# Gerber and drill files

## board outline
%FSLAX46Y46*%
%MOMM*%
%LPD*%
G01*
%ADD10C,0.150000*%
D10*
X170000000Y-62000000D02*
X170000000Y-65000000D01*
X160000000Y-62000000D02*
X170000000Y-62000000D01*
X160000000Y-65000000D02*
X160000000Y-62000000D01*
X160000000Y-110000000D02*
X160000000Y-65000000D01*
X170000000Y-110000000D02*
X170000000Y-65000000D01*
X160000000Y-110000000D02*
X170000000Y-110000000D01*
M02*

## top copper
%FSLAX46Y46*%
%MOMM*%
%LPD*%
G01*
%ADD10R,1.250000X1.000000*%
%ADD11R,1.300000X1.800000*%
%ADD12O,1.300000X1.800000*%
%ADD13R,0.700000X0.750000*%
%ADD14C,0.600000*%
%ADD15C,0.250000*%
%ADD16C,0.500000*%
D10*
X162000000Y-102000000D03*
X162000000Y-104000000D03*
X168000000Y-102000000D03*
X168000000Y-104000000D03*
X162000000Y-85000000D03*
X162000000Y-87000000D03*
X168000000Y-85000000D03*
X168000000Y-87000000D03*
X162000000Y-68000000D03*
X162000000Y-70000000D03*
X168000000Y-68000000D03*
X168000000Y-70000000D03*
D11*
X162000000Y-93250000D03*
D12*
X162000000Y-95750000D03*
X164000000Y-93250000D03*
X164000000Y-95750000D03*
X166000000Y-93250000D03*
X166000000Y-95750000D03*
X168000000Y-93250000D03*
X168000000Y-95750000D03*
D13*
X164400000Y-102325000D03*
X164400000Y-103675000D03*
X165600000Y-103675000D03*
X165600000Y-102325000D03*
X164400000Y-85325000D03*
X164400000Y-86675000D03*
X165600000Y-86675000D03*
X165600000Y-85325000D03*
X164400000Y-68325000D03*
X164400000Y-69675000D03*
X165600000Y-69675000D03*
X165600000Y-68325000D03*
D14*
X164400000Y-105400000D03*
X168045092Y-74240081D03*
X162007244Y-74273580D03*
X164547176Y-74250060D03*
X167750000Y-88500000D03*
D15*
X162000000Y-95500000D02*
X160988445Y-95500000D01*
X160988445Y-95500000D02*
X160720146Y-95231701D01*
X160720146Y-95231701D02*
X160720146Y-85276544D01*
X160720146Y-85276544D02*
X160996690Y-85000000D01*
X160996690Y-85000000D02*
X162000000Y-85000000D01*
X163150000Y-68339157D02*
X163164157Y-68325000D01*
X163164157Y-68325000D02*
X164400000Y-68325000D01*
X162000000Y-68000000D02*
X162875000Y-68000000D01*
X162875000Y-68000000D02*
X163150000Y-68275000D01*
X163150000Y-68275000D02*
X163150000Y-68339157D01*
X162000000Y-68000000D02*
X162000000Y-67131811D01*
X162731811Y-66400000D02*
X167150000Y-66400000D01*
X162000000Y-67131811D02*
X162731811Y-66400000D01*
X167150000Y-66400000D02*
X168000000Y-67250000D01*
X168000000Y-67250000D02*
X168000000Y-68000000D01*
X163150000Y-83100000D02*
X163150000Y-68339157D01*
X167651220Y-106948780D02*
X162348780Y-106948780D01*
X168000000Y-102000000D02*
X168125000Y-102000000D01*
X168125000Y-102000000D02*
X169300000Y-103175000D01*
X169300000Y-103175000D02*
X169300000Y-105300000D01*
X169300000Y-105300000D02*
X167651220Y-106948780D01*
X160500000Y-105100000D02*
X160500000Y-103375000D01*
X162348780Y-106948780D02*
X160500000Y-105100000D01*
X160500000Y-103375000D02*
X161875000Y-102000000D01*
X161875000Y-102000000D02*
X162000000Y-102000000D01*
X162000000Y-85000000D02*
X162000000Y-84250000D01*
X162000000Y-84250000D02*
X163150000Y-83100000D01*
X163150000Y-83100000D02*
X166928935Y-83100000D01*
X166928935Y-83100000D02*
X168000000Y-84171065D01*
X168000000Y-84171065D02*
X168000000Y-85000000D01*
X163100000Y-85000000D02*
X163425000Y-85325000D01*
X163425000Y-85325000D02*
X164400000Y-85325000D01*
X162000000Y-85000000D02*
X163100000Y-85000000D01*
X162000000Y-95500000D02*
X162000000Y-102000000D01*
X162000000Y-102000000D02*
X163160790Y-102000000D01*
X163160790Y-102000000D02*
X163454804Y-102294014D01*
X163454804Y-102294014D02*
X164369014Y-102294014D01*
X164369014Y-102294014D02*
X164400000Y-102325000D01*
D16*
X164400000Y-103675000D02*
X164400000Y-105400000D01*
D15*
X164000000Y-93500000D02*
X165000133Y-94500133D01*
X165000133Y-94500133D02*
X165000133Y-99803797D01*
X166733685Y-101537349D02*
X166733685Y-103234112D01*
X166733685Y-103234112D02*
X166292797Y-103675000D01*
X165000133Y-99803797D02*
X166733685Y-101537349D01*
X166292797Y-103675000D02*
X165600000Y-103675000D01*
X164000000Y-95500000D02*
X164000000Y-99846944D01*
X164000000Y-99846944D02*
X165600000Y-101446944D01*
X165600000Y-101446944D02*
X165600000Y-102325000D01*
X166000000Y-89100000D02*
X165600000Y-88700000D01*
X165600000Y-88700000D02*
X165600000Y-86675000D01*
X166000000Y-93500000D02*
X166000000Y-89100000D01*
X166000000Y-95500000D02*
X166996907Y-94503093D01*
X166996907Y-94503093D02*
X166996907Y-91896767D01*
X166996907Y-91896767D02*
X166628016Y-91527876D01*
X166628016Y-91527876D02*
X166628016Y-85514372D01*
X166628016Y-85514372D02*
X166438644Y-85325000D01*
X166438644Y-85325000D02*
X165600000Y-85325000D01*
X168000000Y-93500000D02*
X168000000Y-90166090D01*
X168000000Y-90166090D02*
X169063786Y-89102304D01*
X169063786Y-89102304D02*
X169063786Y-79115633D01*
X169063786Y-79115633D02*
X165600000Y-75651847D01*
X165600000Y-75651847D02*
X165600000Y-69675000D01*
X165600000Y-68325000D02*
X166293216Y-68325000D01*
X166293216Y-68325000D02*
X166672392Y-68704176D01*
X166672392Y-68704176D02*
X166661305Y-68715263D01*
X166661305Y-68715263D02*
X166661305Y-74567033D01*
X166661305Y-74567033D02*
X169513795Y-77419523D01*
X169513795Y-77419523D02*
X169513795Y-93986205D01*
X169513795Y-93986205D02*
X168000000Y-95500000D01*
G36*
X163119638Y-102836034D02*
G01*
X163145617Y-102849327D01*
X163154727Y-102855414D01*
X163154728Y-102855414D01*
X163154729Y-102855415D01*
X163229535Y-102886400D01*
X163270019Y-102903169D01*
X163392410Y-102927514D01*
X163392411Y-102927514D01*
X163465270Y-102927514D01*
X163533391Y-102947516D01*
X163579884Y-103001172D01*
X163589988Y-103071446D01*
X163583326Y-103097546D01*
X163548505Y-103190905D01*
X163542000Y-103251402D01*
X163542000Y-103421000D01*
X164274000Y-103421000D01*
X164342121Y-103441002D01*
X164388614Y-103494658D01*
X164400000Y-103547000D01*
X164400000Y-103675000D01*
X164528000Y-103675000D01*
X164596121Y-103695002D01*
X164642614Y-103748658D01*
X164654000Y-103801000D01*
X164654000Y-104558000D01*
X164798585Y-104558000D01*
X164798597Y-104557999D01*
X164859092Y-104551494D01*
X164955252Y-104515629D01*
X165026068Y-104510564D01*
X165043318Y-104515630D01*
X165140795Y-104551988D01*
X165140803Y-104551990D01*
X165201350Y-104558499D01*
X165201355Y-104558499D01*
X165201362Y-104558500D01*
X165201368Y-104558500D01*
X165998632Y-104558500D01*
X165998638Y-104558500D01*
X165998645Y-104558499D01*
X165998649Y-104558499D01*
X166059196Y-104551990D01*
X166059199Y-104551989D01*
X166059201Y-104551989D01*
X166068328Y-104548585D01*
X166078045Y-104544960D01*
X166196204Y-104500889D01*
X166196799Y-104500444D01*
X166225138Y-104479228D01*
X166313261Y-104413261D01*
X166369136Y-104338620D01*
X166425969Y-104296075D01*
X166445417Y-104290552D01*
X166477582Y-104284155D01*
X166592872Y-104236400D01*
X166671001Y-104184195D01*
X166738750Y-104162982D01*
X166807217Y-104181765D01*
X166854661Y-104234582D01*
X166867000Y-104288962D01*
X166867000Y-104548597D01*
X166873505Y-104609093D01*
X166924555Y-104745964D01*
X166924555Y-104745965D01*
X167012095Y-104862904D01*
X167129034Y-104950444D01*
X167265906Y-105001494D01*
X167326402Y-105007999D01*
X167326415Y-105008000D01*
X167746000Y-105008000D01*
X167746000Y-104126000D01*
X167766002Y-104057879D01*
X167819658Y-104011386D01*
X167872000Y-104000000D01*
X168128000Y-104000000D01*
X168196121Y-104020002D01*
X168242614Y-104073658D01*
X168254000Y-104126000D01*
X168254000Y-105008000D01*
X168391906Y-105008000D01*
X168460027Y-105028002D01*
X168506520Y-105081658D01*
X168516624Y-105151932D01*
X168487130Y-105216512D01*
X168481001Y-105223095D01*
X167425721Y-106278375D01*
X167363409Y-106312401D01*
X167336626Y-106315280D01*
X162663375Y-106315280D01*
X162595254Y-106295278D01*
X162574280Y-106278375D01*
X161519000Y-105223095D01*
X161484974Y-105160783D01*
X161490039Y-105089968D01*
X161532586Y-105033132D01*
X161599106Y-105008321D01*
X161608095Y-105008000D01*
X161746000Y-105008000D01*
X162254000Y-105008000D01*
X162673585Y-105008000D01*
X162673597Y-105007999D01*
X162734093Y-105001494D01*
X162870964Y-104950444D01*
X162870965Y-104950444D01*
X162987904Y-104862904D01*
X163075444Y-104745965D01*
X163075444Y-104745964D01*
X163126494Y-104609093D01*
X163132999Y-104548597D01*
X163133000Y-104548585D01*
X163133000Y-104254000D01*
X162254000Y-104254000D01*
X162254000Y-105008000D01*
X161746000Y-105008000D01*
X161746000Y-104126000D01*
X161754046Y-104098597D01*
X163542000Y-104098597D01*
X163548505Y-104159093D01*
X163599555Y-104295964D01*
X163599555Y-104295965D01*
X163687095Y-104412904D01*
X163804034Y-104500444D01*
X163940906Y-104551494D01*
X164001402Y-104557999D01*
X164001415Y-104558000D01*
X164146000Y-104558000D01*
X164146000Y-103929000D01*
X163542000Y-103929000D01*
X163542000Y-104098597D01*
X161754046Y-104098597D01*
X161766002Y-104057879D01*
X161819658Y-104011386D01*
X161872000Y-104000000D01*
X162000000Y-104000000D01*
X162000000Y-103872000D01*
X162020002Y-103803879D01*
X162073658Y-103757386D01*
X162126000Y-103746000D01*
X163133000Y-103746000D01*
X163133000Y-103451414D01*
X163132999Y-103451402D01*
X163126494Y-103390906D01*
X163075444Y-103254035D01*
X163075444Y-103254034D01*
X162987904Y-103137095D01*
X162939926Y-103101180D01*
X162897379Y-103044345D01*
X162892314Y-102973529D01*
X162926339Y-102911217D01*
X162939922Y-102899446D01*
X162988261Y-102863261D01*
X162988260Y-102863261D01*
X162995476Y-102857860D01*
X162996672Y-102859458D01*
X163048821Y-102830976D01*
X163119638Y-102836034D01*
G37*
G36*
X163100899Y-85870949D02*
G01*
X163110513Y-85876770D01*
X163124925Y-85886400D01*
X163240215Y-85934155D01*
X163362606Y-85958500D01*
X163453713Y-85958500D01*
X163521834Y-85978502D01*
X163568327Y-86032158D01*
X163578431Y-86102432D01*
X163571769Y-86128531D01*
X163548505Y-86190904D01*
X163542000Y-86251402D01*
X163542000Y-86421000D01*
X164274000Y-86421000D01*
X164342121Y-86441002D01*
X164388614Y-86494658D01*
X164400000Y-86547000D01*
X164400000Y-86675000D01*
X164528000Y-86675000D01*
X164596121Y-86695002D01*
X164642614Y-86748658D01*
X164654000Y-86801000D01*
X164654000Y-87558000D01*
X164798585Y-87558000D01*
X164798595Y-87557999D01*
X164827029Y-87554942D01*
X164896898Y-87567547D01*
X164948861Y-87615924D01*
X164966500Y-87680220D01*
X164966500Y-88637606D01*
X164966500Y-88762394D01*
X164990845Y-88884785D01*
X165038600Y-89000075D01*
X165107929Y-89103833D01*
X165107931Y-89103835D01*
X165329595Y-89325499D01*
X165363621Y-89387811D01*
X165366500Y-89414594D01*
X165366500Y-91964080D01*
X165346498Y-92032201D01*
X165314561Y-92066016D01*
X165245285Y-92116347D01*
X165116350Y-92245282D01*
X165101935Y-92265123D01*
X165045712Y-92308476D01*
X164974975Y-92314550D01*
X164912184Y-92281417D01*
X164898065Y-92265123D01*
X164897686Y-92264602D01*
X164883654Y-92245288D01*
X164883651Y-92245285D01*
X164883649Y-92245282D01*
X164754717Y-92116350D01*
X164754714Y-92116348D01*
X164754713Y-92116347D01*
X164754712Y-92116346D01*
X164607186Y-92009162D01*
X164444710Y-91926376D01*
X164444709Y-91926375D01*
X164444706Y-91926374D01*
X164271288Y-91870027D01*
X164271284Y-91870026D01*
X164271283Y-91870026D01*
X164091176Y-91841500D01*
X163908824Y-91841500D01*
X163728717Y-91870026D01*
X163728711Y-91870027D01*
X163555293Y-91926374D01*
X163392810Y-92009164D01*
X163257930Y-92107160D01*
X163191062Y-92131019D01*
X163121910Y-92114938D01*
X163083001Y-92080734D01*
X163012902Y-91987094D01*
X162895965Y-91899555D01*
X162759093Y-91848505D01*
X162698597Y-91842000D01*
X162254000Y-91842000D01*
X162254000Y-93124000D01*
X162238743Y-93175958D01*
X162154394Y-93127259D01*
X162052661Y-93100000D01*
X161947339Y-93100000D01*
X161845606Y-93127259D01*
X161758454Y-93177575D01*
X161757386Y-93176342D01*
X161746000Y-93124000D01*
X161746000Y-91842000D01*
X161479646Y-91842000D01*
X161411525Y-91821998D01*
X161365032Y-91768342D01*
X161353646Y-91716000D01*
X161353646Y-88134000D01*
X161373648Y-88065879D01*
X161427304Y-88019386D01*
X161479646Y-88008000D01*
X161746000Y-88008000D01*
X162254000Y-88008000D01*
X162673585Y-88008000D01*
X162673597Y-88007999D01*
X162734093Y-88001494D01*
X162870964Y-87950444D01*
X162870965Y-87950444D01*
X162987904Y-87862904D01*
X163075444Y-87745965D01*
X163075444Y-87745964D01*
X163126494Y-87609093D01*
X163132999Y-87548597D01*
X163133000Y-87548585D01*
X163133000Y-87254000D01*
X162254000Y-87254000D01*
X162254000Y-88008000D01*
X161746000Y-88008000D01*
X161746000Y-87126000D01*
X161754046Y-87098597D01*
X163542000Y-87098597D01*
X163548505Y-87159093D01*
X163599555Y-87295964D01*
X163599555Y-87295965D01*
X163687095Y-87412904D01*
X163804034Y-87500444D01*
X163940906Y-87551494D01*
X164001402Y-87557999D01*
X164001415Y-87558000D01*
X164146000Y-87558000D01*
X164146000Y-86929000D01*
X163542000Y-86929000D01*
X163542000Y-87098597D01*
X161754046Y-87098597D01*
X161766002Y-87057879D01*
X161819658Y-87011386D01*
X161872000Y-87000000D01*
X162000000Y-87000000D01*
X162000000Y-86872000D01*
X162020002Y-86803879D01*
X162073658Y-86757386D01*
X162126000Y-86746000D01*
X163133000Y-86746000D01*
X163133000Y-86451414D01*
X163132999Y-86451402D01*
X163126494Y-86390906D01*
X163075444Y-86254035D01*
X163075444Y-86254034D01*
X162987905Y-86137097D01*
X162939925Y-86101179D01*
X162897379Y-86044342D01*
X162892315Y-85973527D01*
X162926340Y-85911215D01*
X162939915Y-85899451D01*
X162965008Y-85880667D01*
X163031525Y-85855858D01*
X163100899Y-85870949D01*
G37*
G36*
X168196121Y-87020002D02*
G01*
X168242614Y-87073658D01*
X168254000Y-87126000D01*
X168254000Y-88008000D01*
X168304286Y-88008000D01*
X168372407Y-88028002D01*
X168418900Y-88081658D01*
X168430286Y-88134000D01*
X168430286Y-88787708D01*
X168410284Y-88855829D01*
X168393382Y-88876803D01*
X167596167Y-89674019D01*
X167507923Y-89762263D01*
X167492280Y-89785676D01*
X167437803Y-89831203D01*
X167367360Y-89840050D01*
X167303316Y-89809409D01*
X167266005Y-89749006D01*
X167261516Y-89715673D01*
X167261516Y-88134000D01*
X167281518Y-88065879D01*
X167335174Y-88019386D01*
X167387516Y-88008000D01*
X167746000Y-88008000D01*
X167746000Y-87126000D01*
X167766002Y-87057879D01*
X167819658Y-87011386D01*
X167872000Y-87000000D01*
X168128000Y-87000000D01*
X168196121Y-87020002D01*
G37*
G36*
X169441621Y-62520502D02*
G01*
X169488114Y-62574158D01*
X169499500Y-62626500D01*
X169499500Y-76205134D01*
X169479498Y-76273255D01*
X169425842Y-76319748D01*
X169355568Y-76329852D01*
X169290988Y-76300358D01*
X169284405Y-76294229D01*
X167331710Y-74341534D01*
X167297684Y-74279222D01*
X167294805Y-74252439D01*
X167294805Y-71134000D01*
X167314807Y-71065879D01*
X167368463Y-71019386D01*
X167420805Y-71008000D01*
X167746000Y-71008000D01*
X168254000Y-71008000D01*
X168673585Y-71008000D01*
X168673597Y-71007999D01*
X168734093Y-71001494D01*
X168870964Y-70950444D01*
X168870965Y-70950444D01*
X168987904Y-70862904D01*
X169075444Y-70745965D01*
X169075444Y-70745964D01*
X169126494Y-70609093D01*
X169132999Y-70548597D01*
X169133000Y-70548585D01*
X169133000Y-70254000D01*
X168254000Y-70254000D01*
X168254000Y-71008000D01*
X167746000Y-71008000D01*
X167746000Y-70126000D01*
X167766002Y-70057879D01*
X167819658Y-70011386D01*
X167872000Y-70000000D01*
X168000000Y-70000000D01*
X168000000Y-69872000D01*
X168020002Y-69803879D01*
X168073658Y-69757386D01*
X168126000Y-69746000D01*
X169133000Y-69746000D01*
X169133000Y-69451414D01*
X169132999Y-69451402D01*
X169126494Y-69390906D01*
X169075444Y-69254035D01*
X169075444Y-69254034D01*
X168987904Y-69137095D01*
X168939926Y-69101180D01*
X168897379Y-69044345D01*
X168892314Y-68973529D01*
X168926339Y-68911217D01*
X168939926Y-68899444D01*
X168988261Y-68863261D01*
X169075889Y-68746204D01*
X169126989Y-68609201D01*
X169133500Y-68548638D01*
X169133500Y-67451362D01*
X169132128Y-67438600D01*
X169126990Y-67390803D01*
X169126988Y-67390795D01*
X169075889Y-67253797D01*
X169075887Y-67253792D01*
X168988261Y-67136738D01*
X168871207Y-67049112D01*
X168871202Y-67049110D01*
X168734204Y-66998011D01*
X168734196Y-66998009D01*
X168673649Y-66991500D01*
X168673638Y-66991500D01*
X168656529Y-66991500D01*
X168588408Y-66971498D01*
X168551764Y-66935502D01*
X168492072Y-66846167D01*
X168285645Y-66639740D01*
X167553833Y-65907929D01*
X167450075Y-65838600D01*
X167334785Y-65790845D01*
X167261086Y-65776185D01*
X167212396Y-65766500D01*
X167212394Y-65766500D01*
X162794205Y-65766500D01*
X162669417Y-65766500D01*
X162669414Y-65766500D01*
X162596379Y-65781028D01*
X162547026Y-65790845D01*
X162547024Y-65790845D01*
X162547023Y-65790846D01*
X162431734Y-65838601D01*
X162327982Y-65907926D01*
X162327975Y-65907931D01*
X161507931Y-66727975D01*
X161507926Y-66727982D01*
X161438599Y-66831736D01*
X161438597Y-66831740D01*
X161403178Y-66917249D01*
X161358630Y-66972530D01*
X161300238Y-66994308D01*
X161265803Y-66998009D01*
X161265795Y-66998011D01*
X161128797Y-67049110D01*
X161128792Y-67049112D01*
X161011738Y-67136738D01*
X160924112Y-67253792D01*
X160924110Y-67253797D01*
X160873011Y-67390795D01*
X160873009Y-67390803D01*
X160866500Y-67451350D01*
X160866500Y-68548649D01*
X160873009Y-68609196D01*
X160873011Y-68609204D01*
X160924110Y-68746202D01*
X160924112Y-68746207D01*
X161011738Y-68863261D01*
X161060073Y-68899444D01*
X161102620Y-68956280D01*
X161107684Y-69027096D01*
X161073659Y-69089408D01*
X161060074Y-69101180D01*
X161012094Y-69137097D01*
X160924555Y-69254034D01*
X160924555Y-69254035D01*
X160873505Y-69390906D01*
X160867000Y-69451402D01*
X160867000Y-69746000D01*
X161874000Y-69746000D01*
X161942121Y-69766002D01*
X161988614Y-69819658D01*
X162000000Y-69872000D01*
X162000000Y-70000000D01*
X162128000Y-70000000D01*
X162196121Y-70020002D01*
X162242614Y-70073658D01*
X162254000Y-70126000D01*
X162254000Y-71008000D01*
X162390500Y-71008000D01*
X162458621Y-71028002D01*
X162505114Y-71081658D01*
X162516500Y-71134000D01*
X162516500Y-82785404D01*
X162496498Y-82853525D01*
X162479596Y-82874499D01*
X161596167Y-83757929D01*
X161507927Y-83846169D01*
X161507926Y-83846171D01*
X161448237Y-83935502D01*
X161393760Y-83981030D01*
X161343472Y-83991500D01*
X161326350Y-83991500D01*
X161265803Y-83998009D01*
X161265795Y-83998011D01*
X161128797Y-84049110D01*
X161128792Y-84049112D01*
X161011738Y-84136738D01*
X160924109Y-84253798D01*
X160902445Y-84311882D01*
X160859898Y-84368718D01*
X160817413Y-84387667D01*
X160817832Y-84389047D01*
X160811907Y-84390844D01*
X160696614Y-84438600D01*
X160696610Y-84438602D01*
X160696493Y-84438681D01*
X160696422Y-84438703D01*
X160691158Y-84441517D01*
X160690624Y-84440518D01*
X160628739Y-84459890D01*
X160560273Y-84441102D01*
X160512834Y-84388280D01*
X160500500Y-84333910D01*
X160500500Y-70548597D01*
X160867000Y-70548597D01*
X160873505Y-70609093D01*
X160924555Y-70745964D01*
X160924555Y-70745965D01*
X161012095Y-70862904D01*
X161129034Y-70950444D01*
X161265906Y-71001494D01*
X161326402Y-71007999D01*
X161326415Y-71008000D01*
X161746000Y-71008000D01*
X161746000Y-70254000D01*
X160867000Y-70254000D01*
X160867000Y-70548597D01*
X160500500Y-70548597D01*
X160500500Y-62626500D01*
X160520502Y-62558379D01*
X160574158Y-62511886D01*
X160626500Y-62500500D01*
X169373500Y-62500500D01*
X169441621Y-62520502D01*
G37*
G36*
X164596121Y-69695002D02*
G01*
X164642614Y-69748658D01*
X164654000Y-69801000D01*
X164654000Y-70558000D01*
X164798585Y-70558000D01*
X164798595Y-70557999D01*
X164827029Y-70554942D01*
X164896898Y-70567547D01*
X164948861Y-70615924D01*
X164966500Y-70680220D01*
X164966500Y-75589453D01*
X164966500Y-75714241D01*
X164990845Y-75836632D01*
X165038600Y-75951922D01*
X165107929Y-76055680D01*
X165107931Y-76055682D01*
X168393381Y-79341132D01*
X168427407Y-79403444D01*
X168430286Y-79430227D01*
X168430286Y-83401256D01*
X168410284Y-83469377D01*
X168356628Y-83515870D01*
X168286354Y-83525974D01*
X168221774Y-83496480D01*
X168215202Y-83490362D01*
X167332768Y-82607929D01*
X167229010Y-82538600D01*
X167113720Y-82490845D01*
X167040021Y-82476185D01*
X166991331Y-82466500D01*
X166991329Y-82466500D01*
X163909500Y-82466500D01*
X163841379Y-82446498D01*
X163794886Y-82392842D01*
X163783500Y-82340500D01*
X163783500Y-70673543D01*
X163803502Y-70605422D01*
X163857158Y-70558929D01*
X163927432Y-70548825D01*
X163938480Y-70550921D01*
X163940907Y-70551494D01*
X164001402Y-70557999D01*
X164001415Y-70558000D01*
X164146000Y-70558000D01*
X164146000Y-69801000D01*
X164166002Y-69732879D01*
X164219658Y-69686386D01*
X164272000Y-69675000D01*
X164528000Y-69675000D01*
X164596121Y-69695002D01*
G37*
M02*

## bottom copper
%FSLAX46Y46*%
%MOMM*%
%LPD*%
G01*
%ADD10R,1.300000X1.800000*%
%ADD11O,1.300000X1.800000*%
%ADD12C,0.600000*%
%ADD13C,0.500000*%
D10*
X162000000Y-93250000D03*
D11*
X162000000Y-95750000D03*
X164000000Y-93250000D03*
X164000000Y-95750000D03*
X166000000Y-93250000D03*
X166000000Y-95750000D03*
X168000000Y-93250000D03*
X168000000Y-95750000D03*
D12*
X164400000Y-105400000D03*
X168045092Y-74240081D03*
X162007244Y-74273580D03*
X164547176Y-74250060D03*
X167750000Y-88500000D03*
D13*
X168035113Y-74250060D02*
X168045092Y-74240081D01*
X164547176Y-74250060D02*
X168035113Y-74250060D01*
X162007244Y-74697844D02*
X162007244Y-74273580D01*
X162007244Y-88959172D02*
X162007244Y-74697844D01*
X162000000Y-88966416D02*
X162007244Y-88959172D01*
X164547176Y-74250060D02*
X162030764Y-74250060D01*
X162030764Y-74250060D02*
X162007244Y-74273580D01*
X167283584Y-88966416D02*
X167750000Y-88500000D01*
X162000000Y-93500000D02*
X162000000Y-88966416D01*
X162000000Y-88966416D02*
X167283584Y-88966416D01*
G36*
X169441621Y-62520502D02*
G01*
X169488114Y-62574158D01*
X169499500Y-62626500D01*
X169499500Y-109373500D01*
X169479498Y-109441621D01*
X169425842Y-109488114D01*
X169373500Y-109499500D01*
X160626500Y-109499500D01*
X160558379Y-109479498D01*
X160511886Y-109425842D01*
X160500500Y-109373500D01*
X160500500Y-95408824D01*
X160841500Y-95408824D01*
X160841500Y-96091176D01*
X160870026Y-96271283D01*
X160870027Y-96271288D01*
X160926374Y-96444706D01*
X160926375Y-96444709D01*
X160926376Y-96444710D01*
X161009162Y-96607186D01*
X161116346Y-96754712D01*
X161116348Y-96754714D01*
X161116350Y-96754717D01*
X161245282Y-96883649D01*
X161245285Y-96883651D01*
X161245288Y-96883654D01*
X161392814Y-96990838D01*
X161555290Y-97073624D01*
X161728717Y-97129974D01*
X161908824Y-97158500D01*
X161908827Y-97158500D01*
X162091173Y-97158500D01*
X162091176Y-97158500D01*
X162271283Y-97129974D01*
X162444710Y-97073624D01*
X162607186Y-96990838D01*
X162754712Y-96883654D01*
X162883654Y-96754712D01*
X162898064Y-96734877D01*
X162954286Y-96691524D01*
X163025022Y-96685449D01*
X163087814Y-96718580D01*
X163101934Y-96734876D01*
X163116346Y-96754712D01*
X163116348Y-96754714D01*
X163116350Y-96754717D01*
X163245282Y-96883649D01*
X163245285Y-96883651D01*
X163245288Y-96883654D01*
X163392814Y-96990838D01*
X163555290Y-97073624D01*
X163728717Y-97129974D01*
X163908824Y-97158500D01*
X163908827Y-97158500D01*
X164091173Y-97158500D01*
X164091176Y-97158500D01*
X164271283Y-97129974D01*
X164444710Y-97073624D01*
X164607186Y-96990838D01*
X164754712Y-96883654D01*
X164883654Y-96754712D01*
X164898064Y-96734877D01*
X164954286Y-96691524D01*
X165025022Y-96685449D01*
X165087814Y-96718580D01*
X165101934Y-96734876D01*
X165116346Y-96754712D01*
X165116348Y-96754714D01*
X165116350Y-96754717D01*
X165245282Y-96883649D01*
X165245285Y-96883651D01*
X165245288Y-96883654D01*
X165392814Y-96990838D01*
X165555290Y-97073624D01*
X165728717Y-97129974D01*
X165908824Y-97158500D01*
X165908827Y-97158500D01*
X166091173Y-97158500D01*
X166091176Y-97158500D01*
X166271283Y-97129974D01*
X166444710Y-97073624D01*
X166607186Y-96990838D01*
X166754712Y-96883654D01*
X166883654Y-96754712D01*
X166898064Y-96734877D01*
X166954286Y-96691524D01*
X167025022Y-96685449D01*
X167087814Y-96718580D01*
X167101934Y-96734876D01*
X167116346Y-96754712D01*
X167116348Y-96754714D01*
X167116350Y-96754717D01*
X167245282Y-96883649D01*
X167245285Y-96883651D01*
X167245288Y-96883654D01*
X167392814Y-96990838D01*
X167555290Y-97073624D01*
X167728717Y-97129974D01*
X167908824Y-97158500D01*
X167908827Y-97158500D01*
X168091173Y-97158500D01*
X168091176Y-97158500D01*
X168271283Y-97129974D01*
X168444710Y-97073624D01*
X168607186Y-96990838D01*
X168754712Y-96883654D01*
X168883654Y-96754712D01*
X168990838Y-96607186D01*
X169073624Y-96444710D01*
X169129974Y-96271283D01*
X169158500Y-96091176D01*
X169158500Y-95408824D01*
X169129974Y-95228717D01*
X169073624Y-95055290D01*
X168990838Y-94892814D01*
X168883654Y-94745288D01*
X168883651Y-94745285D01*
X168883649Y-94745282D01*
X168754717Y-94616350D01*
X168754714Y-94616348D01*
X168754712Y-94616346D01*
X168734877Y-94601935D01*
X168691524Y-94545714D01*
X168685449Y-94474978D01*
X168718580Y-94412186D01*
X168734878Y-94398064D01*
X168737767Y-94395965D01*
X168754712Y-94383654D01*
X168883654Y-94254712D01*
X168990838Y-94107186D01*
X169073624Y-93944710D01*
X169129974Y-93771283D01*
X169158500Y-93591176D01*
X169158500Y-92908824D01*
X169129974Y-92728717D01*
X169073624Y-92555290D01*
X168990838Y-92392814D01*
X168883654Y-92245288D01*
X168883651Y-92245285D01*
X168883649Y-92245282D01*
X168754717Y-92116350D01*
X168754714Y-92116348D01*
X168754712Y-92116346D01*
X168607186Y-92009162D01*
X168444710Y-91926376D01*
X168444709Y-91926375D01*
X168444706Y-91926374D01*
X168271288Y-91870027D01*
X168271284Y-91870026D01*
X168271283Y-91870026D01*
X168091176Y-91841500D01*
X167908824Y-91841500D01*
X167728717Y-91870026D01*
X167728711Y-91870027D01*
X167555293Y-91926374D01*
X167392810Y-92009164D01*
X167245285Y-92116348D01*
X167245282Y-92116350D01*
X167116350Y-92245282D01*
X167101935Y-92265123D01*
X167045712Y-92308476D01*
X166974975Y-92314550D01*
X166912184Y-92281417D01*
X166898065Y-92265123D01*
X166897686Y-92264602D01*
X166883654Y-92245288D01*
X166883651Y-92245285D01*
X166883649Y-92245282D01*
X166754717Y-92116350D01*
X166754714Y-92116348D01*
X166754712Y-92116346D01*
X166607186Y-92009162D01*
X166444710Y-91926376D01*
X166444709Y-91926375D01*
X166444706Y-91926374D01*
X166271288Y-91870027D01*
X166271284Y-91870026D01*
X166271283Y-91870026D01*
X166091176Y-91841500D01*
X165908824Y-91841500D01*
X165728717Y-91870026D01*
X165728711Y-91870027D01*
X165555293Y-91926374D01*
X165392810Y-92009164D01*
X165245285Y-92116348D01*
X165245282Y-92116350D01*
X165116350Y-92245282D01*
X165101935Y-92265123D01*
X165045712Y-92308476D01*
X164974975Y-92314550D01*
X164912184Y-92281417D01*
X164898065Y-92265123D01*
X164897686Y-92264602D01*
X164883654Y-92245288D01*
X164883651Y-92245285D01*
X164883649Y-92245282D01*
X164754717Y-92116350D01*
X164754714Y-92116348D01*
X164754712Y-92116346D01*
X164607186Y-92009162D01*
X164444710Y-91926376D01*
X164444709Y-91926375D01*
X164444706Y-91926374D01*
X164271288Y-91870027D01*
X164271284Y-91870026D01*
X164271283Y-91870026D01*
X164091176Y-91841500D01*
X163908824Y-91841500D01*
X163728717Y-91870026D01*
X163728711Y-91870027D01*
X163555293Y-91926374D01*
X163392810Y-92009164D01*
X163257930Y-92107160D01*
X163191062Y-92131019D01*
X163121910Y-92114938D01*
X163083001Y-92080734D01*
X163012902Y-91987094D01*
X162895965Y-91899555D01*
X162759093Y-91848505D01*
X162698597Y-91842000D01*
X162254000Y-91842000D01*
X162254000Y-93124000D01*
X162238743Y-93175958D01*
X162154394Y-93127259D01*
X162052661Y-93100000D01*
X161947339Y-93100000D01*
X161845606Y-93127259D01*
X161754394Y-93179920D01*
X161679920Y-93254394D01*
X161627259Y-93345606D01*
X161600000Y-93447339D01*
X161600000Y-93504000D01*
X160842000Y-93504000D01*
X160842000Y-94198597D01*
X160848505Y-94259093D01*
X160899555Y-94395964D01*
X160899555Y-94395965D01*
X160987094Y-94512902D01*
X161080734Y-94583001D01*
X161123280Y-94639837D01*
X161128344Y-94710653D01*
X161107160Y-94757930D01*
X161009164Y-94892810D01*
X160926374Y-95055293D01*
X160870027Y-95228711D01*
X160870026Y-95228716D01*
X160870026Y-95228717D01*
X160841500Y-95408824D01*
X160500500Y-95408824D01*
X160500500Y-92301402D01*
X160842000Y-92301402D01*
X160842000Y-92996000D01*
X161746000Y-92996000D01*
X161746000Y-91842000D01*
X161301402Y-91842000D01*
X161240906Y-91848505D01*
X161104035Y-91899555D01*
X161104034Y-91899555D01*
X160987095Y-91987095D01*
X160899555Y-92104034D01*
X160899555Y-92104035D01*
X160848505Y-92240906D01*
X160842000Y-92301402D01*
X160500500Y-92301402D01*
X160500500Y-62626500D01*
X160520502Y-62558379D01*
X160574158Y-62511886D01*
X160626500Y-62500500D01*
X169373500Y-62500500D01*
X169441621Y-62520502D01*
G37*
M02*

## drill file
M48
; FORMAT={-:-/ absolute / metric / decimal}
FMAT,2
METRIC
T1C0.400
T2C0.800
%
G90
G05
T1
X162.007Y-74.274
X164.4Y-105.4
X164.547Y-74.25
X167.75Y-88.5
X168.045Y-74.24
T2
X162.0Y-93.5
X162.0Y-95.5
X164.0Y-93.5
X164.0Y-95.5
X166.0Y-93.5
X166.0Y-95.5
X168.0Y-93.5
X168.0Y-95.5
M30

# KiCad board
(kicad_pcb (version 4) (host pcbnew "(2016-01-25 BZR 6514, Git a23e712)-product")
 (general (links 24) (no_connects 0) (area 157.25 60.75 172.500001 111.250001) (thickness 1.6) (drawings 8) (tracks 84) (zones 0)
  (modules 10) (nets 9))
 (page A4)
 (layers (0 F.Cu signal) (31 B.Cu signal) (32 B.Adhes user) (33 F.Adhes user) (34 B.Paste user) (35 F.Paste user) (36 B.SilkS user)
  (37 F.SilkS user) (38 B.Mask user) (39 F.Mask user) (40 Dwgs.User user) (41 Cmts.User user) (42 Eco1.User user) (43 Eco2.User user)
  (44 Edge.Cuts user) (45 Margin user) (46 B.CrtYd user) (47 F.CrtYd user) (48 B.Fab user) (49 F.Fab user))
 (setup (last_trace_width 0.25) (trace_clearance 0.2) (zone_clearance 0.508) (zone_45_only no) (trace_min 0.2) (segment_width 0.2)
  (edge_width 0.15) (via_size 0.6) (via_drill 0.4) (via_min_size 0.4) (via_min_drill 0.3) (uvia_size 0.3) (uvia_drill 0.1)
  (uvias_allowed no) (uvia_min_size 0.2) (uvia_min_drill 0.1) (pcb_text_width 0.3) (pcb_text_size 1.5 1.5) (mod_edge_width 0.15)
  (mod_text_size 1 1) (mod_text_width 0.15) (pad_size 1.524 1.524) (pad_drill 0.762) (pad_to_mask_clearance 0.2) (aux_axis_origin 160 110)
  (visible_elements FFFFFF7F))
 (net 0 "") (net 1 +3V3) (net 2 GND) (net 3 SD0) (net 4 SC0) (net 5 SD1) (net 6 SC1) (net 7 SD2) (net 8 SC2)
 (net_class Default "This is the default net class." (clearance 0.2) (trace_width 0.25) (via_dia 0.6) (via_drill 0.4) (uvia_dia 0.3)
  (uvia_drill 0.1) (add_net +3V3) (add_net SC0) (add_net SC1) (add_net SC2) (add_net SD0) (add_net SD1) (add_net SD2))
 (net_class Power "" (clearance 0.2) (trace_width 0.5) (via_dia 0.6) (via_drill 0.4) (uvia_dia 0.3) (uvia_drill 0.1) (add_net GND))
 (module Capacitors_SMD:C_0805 (layer F.Cu) (at 162 103 270)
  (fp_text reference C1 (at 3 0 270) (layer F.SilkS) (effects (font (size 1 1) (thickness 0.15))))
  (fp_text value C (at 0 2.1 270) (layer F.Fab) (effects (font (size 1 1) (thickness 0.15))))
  (pad 1 smd rect (at -1 0 270) (size 1 1.25) (layers F.Cu F.Paste F.Mask) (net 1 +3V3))
  (pad 2 smd rect (at 1 0 270) (size 1 1.25) (layers F.Cu F.Paste F.Mask) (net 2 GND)))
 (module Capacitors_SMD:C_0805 (layer F.Cu) (at 168 103 270)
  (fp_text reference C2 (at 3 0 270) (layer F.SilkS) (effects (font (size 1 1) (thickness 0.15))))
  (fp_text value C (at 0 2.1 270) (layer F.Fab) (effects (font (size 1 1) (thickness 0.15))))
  (pad 1 smd rect (at -1 0 270) (size 1 1.25) (layers F.Cu F.Paste F.Mask) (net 1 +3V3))
  (pad 2 smd rect (at 1 0 270) (size 1 1.25) (layers F.Cu F.Paste F.Mask) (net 2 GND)))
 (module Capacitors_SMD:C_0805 (layer F.Cu) (at 162 86 270)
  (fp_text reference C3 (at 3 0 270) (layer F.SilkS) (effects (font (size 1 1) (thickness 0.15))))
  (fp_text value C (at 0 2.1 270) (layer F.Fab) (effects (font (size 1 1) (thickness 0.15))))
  (pad 1 smd rect (at -1 0 270) (size 1 1.25) (layers F.Cu F.Paste F.Mask) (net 1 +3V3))
  (pad 2 smd rect (at 1 0 270) (size 1 1.25) (layers F.Cu F.Paste F.Mask) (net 2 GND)))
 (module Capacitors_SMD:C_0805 (layer F.Cu) (at 168 86 270)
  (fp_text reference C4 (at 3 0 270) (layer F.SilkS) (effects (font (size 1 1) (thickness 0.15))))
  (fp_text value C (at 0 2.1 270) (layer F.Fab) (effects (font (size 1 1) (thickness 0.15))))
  (pad 1 smd rect (at -1 0 270) (size 1 1.25) (layers F.Cu F.Paste F.Mask) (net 1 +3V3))
  (pad 2 smd rect (at 1 0 270) (size 1 1.25) (layers F.Cu F.Paste F.Mask) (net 2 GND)))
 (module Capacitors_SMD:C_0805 (layer F.Cu) (at 162 69 270)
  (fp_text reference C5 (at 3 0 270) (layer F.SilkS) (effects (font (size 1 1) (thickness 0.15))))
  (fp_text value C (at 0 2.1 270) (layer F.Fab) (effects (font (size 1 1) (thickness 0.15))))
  (pad 1 smd rect (at -1 0 270) (size 1 1.25) (layers F.Cu F.Paste F.Mask) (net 1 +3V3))
  (pad 2 smd rect (at 1 0 270) (size 1 1.25) (layers F.Cu F.Paste F.Mask) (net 2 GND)))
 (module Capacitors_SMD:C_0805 (layer F.Cu) (at 168 69 270)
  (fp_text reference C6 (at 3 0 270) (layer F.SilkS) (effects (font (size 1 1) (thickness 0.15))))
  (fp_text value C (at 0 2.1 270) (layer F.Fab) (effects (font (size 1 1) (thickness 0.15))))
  (pad 1 smd rect (at -1 0 270) (size 1 1.25) (layers F.Cu F.Paste F.Mask) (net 1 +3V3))
  (pad 2 smd rect (at 1 0 270) (size 1 1.25) (layers F.Cu F.Paste F.Mask) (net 2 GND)))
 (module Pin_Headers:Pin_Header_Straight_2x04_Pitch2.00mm (layer B.Cu) (at 165 94.5)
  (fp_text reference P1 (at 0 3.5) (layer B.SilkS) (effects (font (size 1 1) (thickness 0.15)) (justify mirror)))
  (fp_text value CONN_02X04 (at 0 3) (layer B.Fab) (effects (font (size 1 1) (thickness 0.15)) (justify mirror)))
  (pad 1 thru_hole rect (at -3 -1) (size 1.3 1.8) (drill 0.8 (offset 0 -0.25)) (layers *.Cu *.Mask B.SilkS) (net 2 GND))
  (pad 2 thru_hole oval (at -3 1) (size 1.3 1.8) (drill 0.8 (offset 0 0.25)) (layers *.Cu *.Mask B.SilkS) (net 1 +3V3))
  (pad 3 thru_hole oval (at -1 -1) (size 1.3 1.8) (drill 0.8 (offset 0 -0.25)) (layers *.Cu *.Mask B.SilkS) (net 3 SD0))
  (pad 4 thru_hole oval (at -1 1) (size 1.3 1.8) (drill 0.8 (offset 0 0.25)) (layers *.Cu *.Mask B.SilkS) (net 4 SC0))
  (pad 5 thru_hole oval (at 1 -1) (size 1.3 1.8) (drill 0.8 (offset 0 -0.25)) (layers *.Cu *.Mask B.SilkS) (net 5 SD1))
  (pad 6 thru_hole oval (at 1 1) (size 1.3 1.8) (drill 0.8 (offset 0 0.25)) (layers *.Cu *.Mask B.SilkS) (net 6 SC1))
  (pad 7 thru_hole oval (at 3 -1) (size 1.3 1.8) (drill 0.8 (offset 0 -0.25)) (layers *.Cu *.Mask B.SilkS) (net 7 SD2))
  (pad 8 thru_hole oval (at 3 1) (size 1.3 1.8) (drill 0.8 (offset 0 0.25)) (layers *.Cu *.Mask B.SilkS) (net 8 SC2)))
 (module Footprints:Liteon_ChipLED (layer F.Cu) (at 165 103)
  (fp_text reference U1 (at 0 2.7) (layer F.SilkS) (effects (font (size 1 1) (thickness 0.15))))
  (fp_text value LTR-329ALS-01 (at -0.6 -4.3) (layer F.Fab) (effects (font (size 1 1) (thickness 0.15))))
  (pad 1 smd rect (at -0.6 -0.675) (size 0.7 0.75) (layers F.Cu F.Paste F.Mask) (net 1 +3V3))
  (pad 2 smd rect (at -0.6 0.675) (size 0.7 0.75) (layers F.Cu F.Paste F.Mask) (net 2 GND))
  (pad 3 smd rect (at 0.6 0.675) (size 0.7 0.75) (layers F.Cu F.Paste F.Mask) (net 3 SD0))
  (pad 4 smd rect (at 0.6 -0.675) (size 0.7 0.75) (layers F.Cu F.Paste F.Mask) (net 4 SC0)))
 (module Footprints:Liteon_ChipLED (layer F.Cu) (at 165 86)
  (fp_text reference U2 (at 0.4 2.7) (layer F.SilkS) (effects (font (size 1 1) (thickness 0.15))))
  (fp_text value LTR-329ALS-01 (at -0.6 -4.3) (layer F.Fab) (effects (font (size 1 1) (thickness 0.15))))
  (pad 1 smd rect (at -0.6 -0.675) (size 0.7 0.75) (layers F.Cu F.Paste F.Mask) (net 1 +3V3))
  (pad 2 smd rect (at -0.6 0.675) (size 0.7 0.75) (layers F.Cu F.Paste F.Mask) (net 2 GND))
  (pad 3 smd rect (at 0.6 0.675) (size 0.7 0.75) (layers F.Cu F.Paste F.Mask) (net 5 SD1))
  (pad 4 smd rect (at 0.6 -0.675) (size 0.7 0.75) (layers F.Cu F.Paste F.Mask) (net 6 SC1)))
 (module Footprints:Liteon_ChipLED (layer F.Cu) (at 165 69)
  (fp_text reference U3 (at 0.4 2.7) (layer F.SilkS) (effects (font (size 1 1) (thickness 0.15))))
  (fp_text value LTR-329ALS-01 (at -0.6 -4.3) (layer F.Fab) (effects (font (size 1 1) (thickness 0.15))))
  (pad 1 smd rect (at -0.6 -0.675) (size 0.7 0.75) (layers F.Cu F.Paste F.Mask) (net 1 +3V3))
  (pad 2 smd rect (at -0.6 0.675) (size 0.7 0.75) (layers F.Cu F.Paste F.Mask) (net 2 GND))
  (pad 3 smd rect (at 0.6 0.675) (size 0.7 0.75) (layers F.Cu F.Paste F.Mask) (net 7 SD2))
  (pad 4 smd rect (at 0.6 -0.675) (size 0.7 0.75) (layers F.Cu F.Paste F.Mask) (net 8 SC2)))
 (gr_line (start 170 62) (end 170 65) (layer Edge.Cuts) (width 0.15))
 (gr_line (start 160 62) (end 170 62) (layer Edge.Cuts) (width 0.15))
 (gr_line (start 160 65) (end 160 62) (layer Edge.Cuts) (width 0.15))
 (gr_line (start 160 110) (end 160 65) (layer Edge.Cuts) (width 0.15))
 (gr_line (start 170 110) (end 170 65) (layer Edge.Cuts) (width 0.15))
 (gr_line (start 160 110) (end 170 110) (layer Edge.Cuts) (width 0.15))
 (segment (start 162 95.5) (end 160.988445 95.5) (width 0.25) (layer F.Cu) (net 1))
 (segment (start 160.988445 95.5) (end 160.720146 95.231701) (width 0.25) (layer F.Cu) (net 1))
 (segment (start 160.720146 95.231701) (end 160.720146 85.276544) (width 0.25) (layer F.Cu) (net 1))
 (segment (start 160.720146 85.276544) (end 160.99669 85) (width 0.25) (layer F.Cu) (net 1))
 (segment (start 160.99669 85) (end 162 85) (width 0.25) (layer F.Cu) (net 1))
 (segment (start 163.15 68.339157) (end 163.164157 68.325) (width 0.25) (layer F.Cu) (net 1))
 (segment (start 163.164157 68.325) (end 164.4 68.325) (width 0.25) (layer F.Cu) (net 1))
 (segment (start 162 68) (end 162.875 68) (width 0.25) (layer F.Cu) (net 1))
 (segment (start 162.875 68) (end 163.15 68.275) (width 0.25) (layer F.Cu) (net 1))
 (segment (start 163.15 68.275) (end 163.15 68.339157) (width 0.25) (layer F.Cu) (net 1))
 (segment (start 162 68) (end 162 67.131811) (width 0.25) (layer F.Cu) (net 1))
 (segment (start 162.731811 66.4) (end 167.15 66.4) (width 0.25) (layer F.Cu) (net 1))
 (segment (start 162 67.131811) (end 162.731811 66.4) (width 0.25) (layer F.Cu) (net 1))
 (segment (start 167.15 66.4) (end 168 67.25) (width 0.25) (layer F.Cu) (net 1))
 (segment (start 168 67.25) (end 168 68) (width 0.25) (layer F.Cu) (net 1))
 (segment (start 163.15 83.1) (end 163.15 68.339157) (width 0.25) (layer F.Cu) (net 1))
 (segment (start 167.65122 106.94878) (end 162.34878 106.94878) (width 0.25) (layer F.Cu) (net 1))
 (segment (start 168 102) (end 168.125 102) (width 0.25) (layer F.Cu) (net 1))
 (segment (start 168.125 102) (end 169.3 103.175) (width 0.25) (layer F.Cu) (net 1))
 (segment (start 169.3 103.175) (end 169.3 105.3) (width 0.25) (layer F.Cu) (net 1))
 (segment (start 169.3 105.3) (end 167.65122 106.94878) (width 0.25) (layer F.Cu) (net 1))
 (segment (start 160.5 105.1) (end 160.5 103.375) (width 0.25) (layer F.Cu) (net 1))
 (segment (start 162.34878 106.94878) (end 160.5 105.1) (width 0.25) (layer F.Cu) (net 1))
 (segment (start 160.5 103.375) (end 161.875 102) (width 0.25) (layer F.Cu) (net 1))
 (segment (start 161.875 102) (end 162 102) (width 0.25) (layer F.Cu) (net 1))
 (segment (start 162 85) (end 162 84.25) (width 0.25) (layer F.Cu) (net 1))
 (segment (start 162 84.25) (end 163.15 83.1) (width 0.25) (layer F.Cu) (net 1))
 (segment (start 163.15 83.1) (end 166.928935 83.1) (width 0.25) (layer F.Cu) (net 1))
 (segment (start 166.928935 83.1) (end 168 84.171065) (width 0.25) (layer F.Cu) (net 1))
 (segment (start 168 84.171065) (end 168 85) (width 0.25) (layer F.Cu) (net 1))
 (segment (start 163.1 85) (end 163.425 85.325) (width 0.25) (layer F.Cu) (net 1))
 (segment (start 163.425 85.325) (end 164.4 85.325) (width 0.25) (layer F.Cu) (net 1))
 (segment (start 162 85) (end 163.1 85) (width 0.25) (layer F.Cu) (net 1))
 (segment (start 162 95.5) (end 162 102) (width 0.25) (layer F.Cu) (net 1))
 (segment (start 162 102) (end 163.16079 102) (width 0.25) (layer F.Cu) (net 1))
 (segment (start 163.16079 102) (end 163.454804 102.294014) (width 0.25) (layer F.Cu) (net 1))
 (segment (start 163.454804 102.294014) (end 164.369014 102.294014) (width 0.25) (layer F.Cu) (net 1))
 (segment (start 164.369014 102.294014) (end 164.4 102.325) (width 0.25) (layer F.Cu) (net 1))
 (via (at 164.4 105.4) (size 0.6) (drill 0.4) (layers F.Cu B.Cu) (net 2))
 (segment (start 164.4 103.675) (end 164.4 105.4) (width 0.5) (layer F.Cu) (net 2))
 (segment (start 168.035113 74.25006) (end 168.045092 74.240081) (width 0.5) (layer B.Cu) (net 2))
 (segment (start 164.547176 74.25006) (end 168.035113 74.25006) (width 0.5) (layer B.Cu) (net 2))
 (via (at 168.045092 74.240081) (size 0.6) (drill 0.4) (layers F.Cu B.Cu) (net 2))
 (segment (start 162.007244 74.697844) (end 162.007244 74.27358) (width 0.5) (layer B.Cu) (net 2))
 (segment (start 162.007244 88.959172) (end 162.007244 74.697844) (width 0.5) (layer B.Cu) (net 2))
 (segment (start 162 88.966416) (end 162.007244 88.959172) (width 0.5) (layer B.Cu) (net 2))
 (segment (start 164.547176 74.25006) (end 162.030764 74.25006) (width 0.5) (layer B.Cu) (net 2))
 (segment (start 162.030764 74.25006) (end 162.007244 74.27358) (width 0.5) (layer B.Cu) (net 2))
 (via (at 162.007244 74.27358) (size 0.6) (drill 0.4) (layers F.Cu B.Cu) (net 2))
 (via (at 164.547176 74.25006) (size 0.6) (drill 0.4) (layers F.Cu B.Cu) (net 2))
 (via (at 167.75 88.5) (size 0.6) (drill 0.4) (layers F.Cu B.Cu) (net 2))
 (segment (start 167.283584 88.966416) (end 167.75 88.5) (width 0.5) (layer B.Cu) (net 2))
 (segment (start 162 93.5) (end 162 88.966416) (width 0.5) (layer B.Cu) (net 2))
 (segment (start 162 88.966416) (end 167.283584 88.966416) (width 0.5) (layer B.Cu) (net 2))
 (segment (start 164 93.5) (end 165.000133 94.500133) (width 0.25) (layer F.Cu) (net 3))
 (segment (start 165.000133 94.500133) (end 165.000133 99.803797) (width 0.25) (layer F.Cu) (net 3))
 (segment (start 166.733685 101.537349) (end 166.733685 103.234112) (width 0.25) (layer F.Cu) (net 3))
 (segment (start 166.733685 103.234112) (end 166.292797 103.675) (width 0.25) (layer F.Cu) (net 3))
 (segment (start 165.000133 99.803797) (end 166.733685 101.537349) (width 0.25) (layer F.Cu) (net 3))
 (segment (start 166.292797 103.675) (end 165.6 103.675) (width 0.25) (layer F.Cu) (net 3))
 (segment (start 164 95.5) (end 164 99.846944) (width 0.25) (layer F.Cu) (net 4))
 (segment (start 164 99.846944) (end 165.6 101.446944) (width 0.25) (layer F.Cu) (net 4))
 (segment (start 165.6 101.446944) (end 165.6 102.325) (width 0.25) (layer F.Cu) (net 4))
 (segment (start 166 89.1) (end 165.6 88.7) (width 0.25) (layer F.Cu) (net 5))
 (segment (start 165.6 88.7) (end 165.6 86.675) (width 0.25) (layer F.Cu) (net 5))
 (segment (start 166 93.5) (end 166 89.1) (width 0.25) (layer F.Cu) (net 5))
 (segment (start 166 95.5) (end 166.996907 94.503093) (width 0.25) (layer F.Cu) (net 6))
 (segment (start 166.996907 94.503093) (end 166.996907 91.896767) (width 0.25) (layer F.Cu) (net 6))
 (segment (start 166.996907 91.896767) (end 166.628016 91.527876) (width 0.25) (layer F.Cu) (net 6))
 (segment (start 166.628016 91.527876) (end 166.628016 85.514372) (width 0.25) (layer F.Cu) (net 6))
 (segment (start 166.628016 85.514372) (end 166.438644 85.325) (width 0.25) (layer F.Cu) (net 6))
 (segment (start 166.438644 85.325) (end 165.6 85.325) (width 0.25) (layer F.Cu) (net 6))
 (segment (start 168 93.5) (end 168 90.16609) (width 0.25) (layer F.Cu) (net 7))
 (segment (start 168 90.16609) (end 169.063786 89.102304) (width 0.25) (layer F.Cu) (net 7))
 (segment (start 169.063786 89.102304) (end 169.063786 79.115633) (width 0.25) (layer F.Cu) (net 7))
 (segment (start 169.063786 79.115633) (end 165.6 75.651847) (width 0.25) (layer F.Cu) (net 7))
 (segment (start 165.6 75.651847) (end 165.6 69.675) (width 0.25) (layer F.Cu) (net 7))
 (segment (start 165.6 68.325) (end 166.293216 68.325) (width 0.25) (layer F.Cu) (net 8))
 (segment (start 166.293216 68.325) (end 166.672392 68.704176) (width 0.25) (layer F.Cu) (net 8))
 (segment (start 166.672392 68.704176) (end 166.661305 68.715263) (width 0.25) (layer F.Cu) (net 8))
 (segment (start 166.661305 68.715263) (end 166.661305 74.567033) (width 0.25) (layer F.Cu) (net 8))
 (segment (start 166.661305 74.567033) (end 169.513795 77.419523) (width 0.25) (layer F.Cu) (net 8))
 (segment (start 169.513795 77.419523) (end 169.513795 93.986205) (width 0.25) (layer F.Cu) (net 8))
 (segment (start 169.513795 93.986205) (end 168 95.5) (width 0.25) (layer F.Cu) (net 8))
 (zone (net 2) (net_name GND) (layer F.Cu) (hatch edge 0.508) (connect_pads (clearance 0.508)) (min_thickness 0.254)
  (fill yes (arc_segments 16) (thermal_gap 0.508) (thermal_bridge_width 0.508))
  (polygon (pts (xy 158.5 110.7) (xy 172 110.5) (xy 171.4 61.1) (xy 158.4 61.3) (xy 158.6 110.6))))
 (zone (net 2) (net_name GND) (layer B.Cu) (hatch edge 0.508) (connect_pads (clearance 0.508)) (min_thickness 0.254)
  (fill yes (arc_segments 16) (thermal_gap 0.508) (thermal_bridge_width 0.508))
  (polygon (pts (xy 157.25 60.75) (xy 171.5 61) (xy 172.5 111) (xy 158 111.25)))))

